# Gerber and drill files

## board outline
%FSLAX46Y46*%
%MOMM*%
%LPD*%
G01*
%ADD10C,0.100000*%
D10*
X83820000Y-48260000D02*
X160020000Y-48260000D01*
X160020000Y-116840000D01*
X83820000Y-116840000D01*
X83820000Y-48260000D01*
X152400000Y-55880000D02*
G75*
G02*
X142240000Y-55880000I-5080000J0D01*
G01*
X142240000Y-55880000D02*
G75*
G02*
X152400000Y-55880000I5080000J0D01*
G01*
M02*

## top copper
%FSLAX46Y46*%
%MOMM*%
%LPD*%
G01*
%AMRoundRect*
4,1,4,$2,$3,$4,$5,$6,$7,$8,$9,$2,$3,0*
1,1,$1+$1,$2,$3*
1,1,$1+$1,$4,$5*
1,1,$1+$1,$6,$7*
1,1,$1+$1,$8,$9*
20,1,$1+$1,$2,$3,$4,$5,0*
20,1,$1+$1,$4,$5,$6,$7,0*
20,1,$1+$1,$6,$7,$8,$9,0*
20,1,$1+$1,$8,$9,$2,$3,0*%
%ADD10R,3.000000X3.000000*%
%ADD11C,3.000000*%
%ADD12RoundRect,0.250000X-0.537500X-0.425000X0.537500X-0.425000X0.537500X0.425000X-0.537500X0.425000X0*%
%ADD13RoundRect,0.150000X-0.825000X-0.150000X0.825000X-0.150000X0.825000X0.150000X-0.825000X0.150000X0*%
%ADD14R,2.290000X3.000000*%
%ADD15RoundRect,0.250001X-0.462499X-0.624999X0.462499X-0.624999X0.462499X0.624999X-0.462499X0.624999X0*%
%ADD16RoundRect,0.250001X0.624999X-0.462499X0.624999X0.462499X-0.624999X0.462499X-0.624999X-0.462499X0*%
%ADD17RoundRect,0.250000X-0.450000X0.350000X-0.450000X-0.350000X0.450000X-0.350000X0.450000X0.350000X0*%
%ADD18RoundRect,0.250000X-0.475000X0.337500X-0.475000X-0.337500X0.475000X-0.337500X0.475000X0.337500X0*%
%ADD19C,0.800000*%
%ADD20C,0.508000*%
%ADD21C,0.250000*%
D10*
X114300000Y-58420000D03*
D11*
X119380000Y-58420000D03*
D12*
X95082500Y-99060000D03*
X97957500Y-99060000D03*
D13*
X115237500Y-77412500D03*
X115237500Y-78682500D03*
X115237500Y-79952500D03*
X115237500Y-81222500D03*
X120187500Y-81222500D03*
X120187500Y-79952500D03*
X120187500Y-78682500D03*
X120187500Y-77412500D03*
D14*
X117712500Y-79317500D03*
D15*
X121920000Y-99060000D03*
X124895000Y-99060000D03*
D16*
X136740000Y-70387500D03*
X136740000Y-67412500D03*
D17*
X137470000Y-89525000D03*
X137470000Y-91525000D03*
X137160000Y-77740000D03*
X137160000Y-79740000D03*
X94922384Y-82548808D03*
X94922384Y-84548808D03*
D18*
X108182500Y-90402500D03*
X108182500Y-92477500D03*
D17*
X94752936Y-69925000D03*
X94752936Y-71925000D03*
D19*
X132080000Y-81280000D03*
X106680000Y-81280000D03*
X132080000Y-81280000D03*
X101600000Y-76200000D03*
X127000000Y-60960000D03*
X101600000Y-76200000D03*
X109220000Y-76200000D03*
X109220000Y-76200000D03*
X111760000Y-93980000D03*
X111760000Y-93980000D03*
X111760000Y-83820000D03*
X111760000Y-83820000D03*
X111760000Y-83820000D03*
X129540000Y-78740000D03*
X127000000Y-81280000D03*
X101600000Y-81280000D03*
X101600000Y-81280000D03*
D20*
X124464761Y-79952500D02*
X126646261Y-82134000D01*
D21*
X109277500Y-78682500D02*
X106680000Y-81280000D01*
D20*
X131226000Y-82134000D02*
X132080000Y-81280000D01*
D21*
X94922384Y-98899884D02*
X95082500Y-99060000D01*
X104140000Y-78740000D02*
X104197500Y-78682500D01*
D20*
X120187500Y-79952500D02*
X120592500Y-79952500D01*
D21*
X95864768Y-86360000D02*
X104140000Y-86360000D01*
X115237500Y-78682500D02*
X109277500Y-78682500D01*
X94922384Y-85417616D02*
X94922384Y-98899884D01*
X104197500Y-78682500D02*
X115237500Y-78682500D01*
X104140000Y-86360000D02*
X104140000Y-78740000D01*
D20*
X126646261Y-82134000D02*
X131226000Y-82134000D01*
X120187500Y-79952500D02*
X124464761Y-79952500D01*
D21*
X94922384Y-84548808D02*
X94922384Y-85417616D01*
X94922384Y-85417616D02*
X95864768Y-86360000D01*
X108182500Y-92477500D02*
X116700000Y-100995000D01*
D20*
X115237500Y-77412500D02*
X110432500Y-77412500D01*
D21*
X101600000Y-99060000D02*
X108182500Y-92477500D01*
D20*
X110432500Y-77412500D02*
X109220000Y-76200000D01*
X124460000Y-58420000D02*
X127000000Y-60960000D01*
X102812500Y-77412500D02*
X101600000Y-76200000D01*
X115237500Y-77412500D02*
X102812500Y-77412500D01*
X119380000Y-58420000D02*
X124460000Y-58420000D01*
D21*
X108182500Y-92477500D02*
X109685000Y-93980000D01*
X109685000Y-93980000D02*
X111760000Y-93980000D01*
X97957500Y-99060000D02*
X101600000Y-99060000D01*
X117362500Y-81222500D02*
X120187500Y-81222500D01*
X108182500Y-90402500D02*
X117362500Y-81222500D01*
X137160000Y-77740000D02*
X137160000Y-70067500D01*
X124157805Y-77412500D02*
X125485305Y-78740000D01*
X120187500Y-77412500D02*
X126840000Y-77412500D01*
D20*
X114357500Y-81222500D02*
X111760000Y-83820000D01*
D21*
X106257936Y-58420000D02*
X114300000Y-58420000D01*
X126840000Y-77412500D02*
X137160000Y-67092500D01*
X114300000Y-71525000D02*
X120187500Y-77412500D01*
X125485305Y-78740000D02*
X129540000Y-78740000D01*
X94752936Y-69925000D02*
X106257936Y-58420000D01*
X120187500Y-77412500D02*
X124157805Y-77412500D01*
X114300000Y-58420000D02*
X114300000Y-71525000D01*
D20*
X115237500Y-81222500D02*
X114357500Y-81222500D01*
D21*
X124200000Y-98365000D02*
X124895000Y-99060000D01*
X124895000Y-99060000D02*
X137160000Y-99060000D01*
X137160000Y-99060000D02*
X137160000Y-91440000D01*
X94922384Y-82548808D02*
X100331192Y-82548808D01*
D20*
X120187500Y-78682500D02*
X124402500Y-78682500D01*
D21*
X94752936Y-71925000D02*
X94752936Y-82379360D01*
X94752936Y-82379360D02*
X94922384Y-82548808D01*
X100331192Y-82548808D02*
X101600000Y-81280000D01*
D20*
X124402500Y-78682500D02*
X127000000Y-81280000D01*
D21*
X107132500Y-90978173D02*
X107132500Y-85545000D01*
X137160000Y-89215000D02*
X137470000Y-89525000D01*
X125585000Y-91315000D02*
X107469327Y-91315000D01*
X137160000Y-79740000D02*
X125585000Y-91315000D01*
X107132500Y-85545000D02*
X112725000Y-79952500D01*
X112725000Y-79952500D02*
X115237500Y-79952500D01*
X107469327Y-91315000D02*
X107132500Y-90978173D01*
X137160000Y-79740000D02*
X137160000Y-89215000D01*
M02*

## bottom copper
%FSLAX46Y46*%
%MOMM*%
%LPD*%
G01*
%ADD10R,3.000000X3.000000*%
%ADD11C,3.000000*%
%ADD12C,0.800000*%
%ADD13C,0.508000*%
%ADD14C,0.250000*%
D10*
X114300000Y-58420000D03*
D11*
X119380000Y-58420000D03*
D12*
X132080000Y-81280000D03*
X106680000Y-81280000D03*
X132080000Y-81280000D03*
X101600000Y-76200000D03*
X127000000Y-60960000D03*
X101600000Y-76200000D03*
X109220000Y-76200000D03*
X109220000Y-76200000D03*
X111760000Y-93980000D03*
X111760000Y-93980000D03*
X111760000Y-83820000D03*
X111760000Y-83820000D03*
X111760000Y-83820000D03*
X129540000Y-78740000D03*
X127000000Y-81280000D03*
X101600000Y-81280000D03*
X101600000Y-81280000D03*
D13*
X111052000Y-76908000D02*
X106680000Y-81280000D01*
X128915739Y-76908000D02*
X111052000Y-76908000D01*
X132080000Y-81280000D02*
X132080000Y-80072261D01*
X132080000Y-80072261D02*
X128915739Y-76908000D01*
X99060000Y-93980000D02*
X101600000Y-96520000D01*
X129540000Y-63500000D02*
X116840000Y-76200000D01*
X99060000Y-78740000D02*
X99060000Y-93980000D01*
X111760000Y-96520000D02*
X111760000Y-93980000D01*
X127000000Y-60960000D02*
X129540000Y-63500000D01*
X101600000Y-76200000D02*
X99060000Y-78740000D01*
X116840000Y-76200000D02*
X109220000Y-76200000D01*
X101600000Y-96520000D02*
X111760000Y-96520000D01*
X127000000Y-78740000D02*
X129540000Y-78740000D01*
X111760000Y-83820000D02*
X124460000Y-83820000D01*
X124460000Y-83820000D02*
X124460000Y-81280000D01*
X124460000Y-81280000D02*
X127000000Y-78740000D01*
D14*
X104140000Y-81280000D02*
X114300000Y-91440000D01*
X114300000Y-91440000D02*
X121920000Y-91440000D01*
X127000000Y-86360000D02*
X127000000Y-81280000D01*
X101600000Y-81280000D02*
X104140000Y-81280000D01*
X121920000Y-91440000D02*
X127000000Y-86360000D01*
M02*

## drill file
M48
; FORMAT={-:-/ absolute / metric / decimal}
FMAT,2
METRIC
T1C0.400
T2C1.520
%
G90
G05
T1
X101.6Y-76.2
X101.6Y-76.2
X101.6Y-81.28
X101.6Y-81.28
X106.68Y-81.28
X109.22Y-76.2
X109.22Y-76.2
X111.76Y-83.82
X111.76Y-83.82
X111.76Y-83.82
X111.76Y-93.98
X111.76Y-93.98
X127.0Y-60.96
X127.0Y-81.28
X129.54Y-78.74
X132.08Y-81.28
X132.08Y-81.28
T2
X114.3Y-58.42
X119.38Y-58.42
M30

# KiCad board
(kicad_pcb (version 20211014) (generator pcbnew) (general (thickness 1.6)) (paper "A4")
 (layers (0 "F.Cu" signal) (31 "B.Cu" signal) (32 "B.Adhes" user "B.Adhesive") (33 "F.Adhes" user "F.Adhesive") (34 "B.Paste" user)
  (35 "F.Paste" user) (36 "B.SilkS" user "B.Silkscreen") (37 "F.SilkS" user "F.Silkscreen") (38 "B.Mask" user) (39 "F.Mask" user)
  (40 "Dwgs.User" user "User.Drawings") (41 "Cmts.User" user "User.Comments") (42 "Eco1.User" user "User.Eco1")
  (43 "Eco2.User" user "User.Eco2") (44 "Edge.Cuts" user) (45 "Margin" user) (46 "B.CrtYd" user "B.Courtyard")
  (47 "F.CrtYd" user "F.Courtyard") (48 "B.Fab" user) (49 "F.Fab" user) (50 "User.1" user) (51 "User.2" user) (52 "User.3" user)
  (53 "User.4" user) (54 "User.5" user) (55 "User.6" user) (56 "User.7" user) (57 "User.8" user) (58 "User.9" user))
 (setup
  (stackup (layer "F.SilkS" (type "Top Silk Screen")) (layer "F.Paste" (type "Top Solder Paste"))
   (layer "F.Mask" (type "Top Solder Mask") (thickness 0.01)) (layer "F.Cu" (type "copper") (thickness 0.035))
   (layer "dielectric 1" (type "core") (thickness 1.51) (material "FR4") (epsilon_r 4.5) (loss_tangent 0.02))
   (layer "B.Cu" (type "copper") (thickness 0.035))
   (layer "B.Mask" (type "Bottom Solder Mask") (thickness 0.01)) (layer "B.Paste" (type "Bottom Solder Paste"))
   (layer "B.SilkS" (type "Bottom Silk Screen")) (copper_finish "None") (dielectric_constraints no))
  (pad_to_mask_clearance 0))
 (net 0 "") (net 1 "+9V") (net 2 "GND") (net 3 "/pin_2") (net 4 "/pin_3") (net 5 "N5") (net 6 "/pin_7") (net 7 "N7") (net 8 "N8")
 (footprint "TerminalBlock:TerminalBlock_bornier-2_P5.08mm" (layer "F.Cu") (at 114.3 58.42)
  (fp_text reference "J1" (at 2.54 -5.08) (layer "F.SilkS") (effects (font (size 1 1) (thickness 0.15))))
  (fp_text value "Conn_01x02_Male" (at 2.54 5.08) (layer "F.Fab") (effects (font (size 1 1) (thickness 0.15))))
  (pad "1" thru_hole rect (at 0 0) (size 3 3) (drill 1.52) (layers *.Cu *.Mask) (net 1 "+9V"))
  (pad "2" thru_hole circle (at 5.08 0) (size 3 3) (drill 1.52) (layers *.Cu *.Mask) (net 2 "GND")))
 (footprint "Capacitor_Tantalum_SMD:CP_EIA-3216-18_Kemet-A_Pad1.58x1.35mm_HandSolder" (layer "F.Cu") (at 96.52 99.06)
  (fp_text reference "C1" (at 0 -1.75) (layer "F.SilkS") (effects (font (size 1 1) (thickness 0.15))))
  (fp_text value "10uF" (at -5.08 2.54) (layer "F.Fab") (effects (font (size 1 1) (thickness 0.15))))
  (pad "1" smd roundrect (at -1.4375 0) (size 1.575 1.35) (layers "F.Cu" "F.Paste" "F.Mask") (roundrect_rratio 0.185185) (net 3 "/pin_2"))
  (pad "2" smd roundrect (at 1.4375 0) (size 1.575 1.35) (layers "F.Cu" "F.Paste" "F.Mask") (roundrect_rratio 0.185185) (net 2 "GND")))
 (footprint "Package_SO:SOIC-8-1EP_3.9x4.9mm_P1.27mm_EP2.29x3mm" (layer "F.Cu") (at 117.7125 79.3175)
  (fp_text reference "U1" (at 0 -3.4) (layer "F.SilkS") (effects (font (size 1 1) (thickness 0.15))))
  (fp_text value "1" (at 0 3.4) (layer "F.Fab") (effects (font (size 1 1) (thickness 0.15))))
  (pad "" smd roundrect (at 0.57 0.75) (size 0.92 1.21) (layers "F.Paste") (roundrect_rratio 0.25))
  (pad "" smd roundrect (at -0.57 -0.75) (size 0.92 1.21) (layers "F.Paste") (roundrect_rratio 0.25))
  (pad "" smd roundrect (at -0.57 0.75) (size 0.92 1.21) (layers "F.Paste") (roundrect_rratio 0.25))
  (pad "" smd roundrect (at 0.57 -0.75) (size 0.92 1.21) (layers "F.Paste") (roundrect_rratio 0.25))
  (pad "1" smd roundrect (at -2.475 -1.905) (size 1.95 0.6) (layers "F.Cu" "F.Paste" "F.Mask") (roundrect_rratio 0.25) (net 2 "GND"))
  (pad "2" smd roundrect (at -2.475 -0.635) (size 1.95 0.6) (layers "F.Cu" "F.Paste" "F.Mask") (roundrect_rratio 0.25) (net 3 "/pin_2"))
  (pad "3" smd roundrect (at -2.475 0.635) (size 1.95 0.6) (layers "F.Cu" "F.Paste" "F.Mask") (roundrect_rratio 0.25) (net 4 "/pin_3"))
  (pad "4" smd roundrect (at -2.475 1.905) (size 1.95 0.6) (layers "F.Cu" "F.Paste" "F.Mask") (roundrect_rratio 0.25) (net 1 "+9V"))
  (pad "5" smd roundrect (at 2.475 1.905) (size 1.95 0.6) (layers "F.Cu" "F.Paste" "F.Mask") (roundrect_rratio 0.25) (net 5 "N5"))
  (pad "6" smd roundrect (at 2.475 0.635) (size 1.95 0.6) (layers "F.Cu" "F.Paste" "F.Mask") (roundrect_rratio 0.25) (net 3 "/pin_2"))
  (pad "7" smd roundrect (at 2.475 -0.635) (size 1.95 0.6) (layers "F.Cu" "F.Paste" "F.Mask") (roundrect_rratio 0.25) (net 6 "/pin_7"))
  (pad "8" smd roundrect (at 2.475 -1.905) (size 1.95 0.6) (layers "F.Cu" "F.Paste" "F.Mask") (roundrect_rratio 0.25) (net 1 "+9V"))
  (pad "9" smd rect (at 0 0) (size 2.29 3) (layers "F.Cu" "F.Mask")))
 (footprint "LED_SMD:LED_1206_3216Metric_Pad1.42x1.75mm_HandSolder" (layer "F.Cu") (at 123.4075 99.06)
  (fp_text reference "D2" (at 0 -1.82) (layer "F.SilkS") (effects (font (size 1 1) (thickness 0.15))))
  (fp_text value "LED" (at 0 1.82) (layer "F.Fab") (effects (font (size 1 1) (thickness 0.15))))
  (pad "1" smd roundrect (at -1.4875 0) (size 1.425 1.75) (layers "F.Cu" "F.Paste" "F.Mask") (roundrect_rratio 0.175439) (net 2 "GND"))
  (pad "2" smd roundrect (at 1.4875 0) (size 1.425 1.75) (layers "F.Cu" "F.Paste" "F.Mask") (roundrect_rratio 0.175439) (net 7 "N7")))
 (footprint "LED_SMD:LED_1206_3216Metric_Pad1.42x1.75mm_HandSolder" (layer "F.Cu") (at 136.74 68.9 90)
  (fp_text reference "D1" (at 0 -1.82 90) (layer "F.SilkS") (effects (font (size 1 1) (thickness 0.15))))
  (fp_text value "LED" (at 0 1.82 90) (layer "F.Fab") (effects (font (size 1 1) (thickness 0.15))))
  (pad "1" smd roundrect (at -1.4875 0 90) (size 1.425 1.75) (layers "F.Cu" "F.Paste" "F.Mask") (roundrect_rratio 0.175439) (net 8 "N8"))
  (pad "2" smd roundrect (at 1.4875 0 90) (size 1.425 1.75) (layers "F.Cu" "F.Paste" "F.Mask") (roundrect_rratio 0.175439) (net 1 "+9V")))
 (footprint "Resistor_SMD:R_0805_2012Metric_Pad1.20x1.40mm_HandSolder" (layer "F.Cu") (at 137.47 90.525 -90)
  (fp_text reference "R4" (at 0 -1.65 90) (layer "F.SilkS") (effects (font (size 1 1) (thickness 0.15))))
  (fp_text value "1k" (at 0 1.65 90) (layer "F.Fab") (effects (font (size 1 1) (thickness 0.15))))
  (pad "1" smd roundrect (at -1 0 270) (size 1.2 1.4) (layers "F.Cu" "F.Paste" "F.Mask") (roundrect_rratio 0.208333) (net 4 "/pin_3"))
  (pad "2" smd roundrect (at 1 0 270) (size 1.2 1.4) (layers "F.Cu" "F.Paste" "F.Mask") (roundrect_rratio 0.208333) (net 7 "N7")))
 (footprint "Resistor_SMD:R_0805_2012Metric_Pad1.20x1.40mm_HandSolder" (layer "F.Cu") (at 137.16 78.74 -90)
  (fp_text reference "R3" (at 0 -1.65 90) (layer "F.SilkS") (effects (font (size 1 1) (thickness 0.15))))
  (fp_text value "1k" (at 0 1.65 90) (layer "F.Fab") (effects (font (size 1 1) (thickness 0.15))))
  (pad "1" smd roundrect (at -1 0 270) (size 1.2 1.4) (layers "F.Cu" "F.Paste" "F.Mask") (roundrect_rratio 0.208333) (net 8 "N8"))
  (pad "2" smd roundrect (at 1 0 270) (size 1.2 1.4) (layers "F.Cu" "F.Paste" "F.Mask") (roundrect_rratio 0.208333) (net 4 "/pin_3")))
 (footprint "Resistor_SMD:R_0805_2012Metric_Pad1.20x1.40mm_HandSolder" (layer "F.Cu") (at 94.922384 83.548808 -90)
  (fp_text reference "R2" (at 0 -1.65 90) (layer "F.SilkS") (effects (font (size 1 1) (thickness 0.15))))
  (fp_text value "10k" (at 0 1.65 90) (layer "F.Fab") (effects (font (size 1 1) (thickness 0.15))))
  (pad "1" smd roundrect (at -1 0 270) (size 1.2 1.4) (layers "F.Cu" "F.Paste" "F.Mask") (roundrect_rratio 0.208333) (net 6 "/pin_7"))
  (pad "2" smd roundrect (at 1 0 270) (size 1.2 1.4) (layers "F.Cu" "F.Paste" "F.Mask") (roundrect_rratio 0.208333) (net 3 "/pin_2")))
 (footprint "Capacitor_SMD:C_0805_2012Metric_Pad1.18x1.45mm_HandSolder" (layer "F.Cu") (at 108.1825 91.44 -90)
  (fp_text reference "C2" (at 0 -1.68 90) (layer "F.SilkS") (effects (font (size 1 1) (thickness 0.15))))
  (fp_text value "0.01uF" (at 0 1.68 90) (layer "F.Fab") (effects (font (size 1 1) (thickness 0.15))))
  (pad "1" smd roundrect (at -1.0375 0 270) (size 1.175 1.45) (layers "F.Cu" "F.Paste" "F.Mask") (roundrect_rratio 0.212766) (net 5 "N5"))
  (pad "2" smd roundrect (at 1.0375 0 270) (size 1.175 1.45) (layers "F.Cu" "F.Paste" "F.Mask") (roundrect_rratio 0.212766) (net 2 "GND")))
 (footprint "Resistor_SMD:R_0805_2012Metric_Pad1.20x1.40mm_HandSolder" (layer "F.Cu") (at 94.752936 70.925 -90)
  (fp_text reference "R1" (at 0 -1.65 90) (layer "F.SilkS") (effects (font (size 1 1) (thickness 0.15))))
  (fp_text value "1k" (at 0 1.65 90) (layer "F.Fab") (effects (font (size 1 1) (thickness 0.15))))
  (pad "1" smd roundrect (at -1 0 270) (size 1.2 1.4) (layers "F.Cu" "F.Paste" "F.Mask") (roundrect_rratio 0.208333) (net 1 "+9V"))
  (pad "2" smd roundrect (at 1 0 270) (size 1.2 1.4) (layers "F.Cu" "F.Paste" "F.Mask") (roundrect_rratio 0.208333) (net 6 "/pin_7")))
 (gr_rect (start 83.82 48.26) (end 160.02 116.84) (layer "Edge.Cuts") (width 0.1) (fill none))
 (gr_circle (center 147.32 55.88) (end 152.4 55.88) (layer "Edge.Cuts") (width 0.1) (fill none))
 (segment (start 124.464761 79.9525) (end 126.646261 82.134) (width 0.508) (layer "F.Cu") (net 3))
 (segment (start 109.2775 78.6825) (end 106.68 81.28) (width 0.25) (layer "F.Cu") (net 3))
 (segment (start 131.226 82.134) (end 132.08 81.28) (width 0.508) (layer "F.Cu") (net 3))
 (segment (start 94.922384 98.899884) (end 95.0825 99.06) (width 0.25) (layer "F.Cu") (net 3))
 (segment (start 104.14 78.74) (end 104.1975 78.6825) (width 0.25) (layer "F.Cu") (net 3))
 (segment (start 120.1875 79.9525) (end 120.5925 79.9525) (width 0.508) (layer "F.Cu") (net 3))
 (segment (start 95.864768 86.36) (end 104.14 86.36) (width 0.25) (layer "F.Cu") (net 3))
 (segment (start 115.2375 78.6825) (end 109.2775 78.6825) (width 0.25) (layer "F.Cu") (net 3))
 (segment (start 94.922384 85.417616) (end 94.922384 98.899884) (width 0.25) (layer "F.Cu") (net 3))
 (segment (start 104.1975 78.6825) (end 115.2375 78.6825) (width 0.25) (layer "F.Cu") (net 3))
 (segment (start 104.14 86.36) (end 104.14 78.74) (width 0.25) (layer "F.Cu") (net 3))
 (segment (start 126.646261 82.134) (end 131.226 82.134) (width 0.508) (layer "F.Cu") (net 3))
 (segment (start 120.1875 79.9525) (end 124.464761 79.9525) (width 0.508) (layer "F.Cu") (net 3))
 (segment (start 94.922384 84.548808) (end 94.922384 85.417616) (width 0.25) (layer "F.Cu") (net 3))
 (segment (start 94.922384 85.417616) (end 95.864768 86.36) (width 0.25) (layer "F.Cu") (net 3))
 (via (at 132.08 81.28) (size 0.8) (drill 0.4) (layers "F.Cu" "B.Cu") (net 3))
 (via (at 106.68 81.28) (size 0.8) (drill 0.4) (layers "F.Cu" "B.Cu") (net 3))
 (via (at 132.08 81.28) (size 0.8) (drill 0.4) (layers "F.Cu" "B.Cu") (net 3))
 (segment (start 111.052 76.908) (end 106.68 81.28) (width 0.508) (layer "B.Cu") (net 3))
 (segment (start 128.915739 76.908) (end 111.052 76.908) (width 0.508) (layer "B.Cu") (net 3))
 (segment (start 132.08 81.28) (end 132.08 80.072261) (width 0.508) (layer "B.Cu") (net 3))
 (segment (start 132.08 80.072261) (end 128.915739 76.908) (width 0.508) (layer "B.Cu") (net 3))
 (segment (start 108.1825 92.4775) (end 116.7 100.995) (width 0.25) (layer "F.Cu") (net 2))
 (segment (start 115.2375 77.4125) (end 110.4325 77.4125) (width 0.508) (layer "F.Cu") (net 2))
 (segment (start 101.6 99.06) (end 108.1825 92.4775) (width 0.25) (layer "F.Cu") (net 2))
 (segment (start 110.4325 77.4125) (end 109.22 76.2) (width 0.508) (layer "F.Cu") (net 2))
 (segment (start 124.46 58.42) (end 127 60.96) (width 0.508) (layer "F.Cu") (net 2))
 (segment (start 102.8125 77.4125) (end 101.6 76.2) (width 0.508) (layer "F.Cu") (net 2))
 (segment (start 115.2375 77.4125) (end 102.8125 77.4125) (width 0.508) (layer "F.Cu") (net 2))
 (segment (start 119.38 58.42) (end 124.46 58.42) (width 0.508) (layer "F.Cu") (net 2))
 (segment (start 108.1825 92.4775) (end 109.685 93.98) (width 0.25) (layer "F.Cu") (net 2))
 (segment (start 109.685 93.98) (end 111.76 93.98) (width 0.25) (layer "F.Cu") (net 2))
 (segment (start 97.9575 99.06) (end 101.6 99.06) (width 0.25) (layer "F.Cu") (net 2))
 (via (at 101.6 76.2) (size 0.8) (drill 0.4) (layers "F.Cu" "B.Cu") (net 2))
 (via (at 127 60.96) (size 0.8) (drill 0.4) (layers "F.Cu" "B.Cu") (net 2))
 (via (at 101.6 76.2) (size 0.8) (drill 0.4) (layers "F.Cu" "B.Cu") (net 2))
 (via (at 109.22 76.2) (size 0.8) (drill 0.4) (layers "F.Cu" "B.Cu") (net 2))
 (via (at 109.22 76.2) (size 0.8) (drill 0.4) (layers "F.Cu" "B.Cu") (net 2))
 (via (at 111.76 93.98) (size 0.8) (drill 0.4) (layers "F.Cu" "B.Cu") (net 2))
 (via (at 111.76 93.98) (size 0.8) (drill 0.4) (layers "F.Cu" "B.Cu") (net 2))
 (segment (start 99.06 93.98) (end 101.6 96.52) (width 0.508) (layer "B.Cu") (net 2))
 (segment (start 129.54 63.5) (end 116.84 76.2) (width 0.508) (layer "B.Cu") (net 2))
 (segment (start 99.06 78.74) (end 99.06 93.98) (width 0.508) (layer "B.Cu") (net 2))
 (segment (start 111.76 96.52) (end 111.76 93.98) (width 0.508) (layer "B.Cu") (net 2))
 (segment (start 127 60.96) (end 129.54 63.5) (width 0.508) (layer "B.Cu") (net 2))
 (segment (start 101.6 76.2) (end 99.06 78.74) (width 0.508) (layer "B.Cu") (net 2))
 (segment (start 116.84 76.2) (end 109.22 76.2) (width 0.508) (layer "B.Cu") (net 2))
 (segment (start 101.6 96.52) (end 111.76 96.52) (width 0.508) (layer "B.Cu") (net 2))
 (segment (start 117.3625 81.2225) (end 120.1875 81.2225) (width 0.25) (layer "F.Cu") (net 5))
 (segment (start 108.1825 90.4025) (end 117.3625 81.2225) (width 0.25) (layer "F.Cu") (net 5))
 (segment (start 137.16 77.74) (end 137.16 70.0675) (width 0.25) (layer "F.Cu") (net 8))
 (segment (start 124.157805 77.4125) (end 125.485305 78.74) (width 0.25) (layer "F.Cu") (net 1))
 (segment (start 120.1875 77.4125) (end 126.84 77.4125) (width 0.25) (layer "F.Cu") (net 1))
 (segment (start 114.3575 81.2225) (end 111.76 83.82) (width 0.508) (layer "F.Cu") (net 1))
 (segment (start 106.257936 58.42) (end 114.3 58.42) (width 0.25) (layer "F.Cu") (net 1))
 (segment (start 126.84 77.4125) (end 137.16 67.0925) (width 0.25) (layer "F.Cu") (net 1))
 (segment (start 114.3 71.525) (end 120.1875 77.4125) (width 0.25) (layer "F.Cu") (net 1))
 (segment (start 125.485305 78.74) (end 129.54 78.74) (width 0.25) (layer "F.Cu") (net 1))
 (segment (start 94.752936 69.925) (end 106.257936 58.42) (width 0.25) (layer "F.Cu") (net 1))
 (segment (start 120.1875 77.4125) (end 124.157805 77.4125) (width 0.25) (layer "F.Cu") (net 1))
 (segment (start 114.3 58.42) (end 114.3 71.525) (width 0.25) (layer "F.Cu") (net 1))
 (segment (start 115.2375 81.2225) (end 114.3575 81.2225) (width 0.508) (layer "F.Cu") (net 1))
 (via (at 111.76 83.82) (size 0.8) (drill 0.4) (layers "F.Cu" "B.Cu") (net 1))
 (via (at 111.76 83.82) (size 0.8) (drill 0.4) (layers "F.Cu" "B.Cu") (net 1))
 (via (at 111.76 83.82) (size 0.8) (drill 0.4) (layers "F.Cu" "B.Cu") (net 1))
 (via (at 129.54 78.74) (size 0.8) (drill 0.4) (layers "F.Cu" "B.Cu") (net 1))
 (segment (start 127 78.74) (end 129.54 78.74) (width 0.508) (layer "B.Cu") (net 1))
 (segment (start 111.76 83.82) (end 124.46 83.82) (width 0.508) (layer "B.Cu") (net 1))
 (segment (start 124.46 83.82) (end 124.46 81.28) (width 0.508) (layer "B.Cu") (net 1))
 (segment (start 124.46 81.28) (end 127 78.74) (width 0.508) (layer "B.Cu") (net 1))
 (segment (start 124.2 98.365) (end 124.895 99.06) (width 0.25) (layer "F.Cu") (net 7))
 (segment (start 124.895 99.06) (end 137.16 99.06) (width 0.25) (layer "F.Cu") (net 7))
 (segment (start 137.16 99.06) (end 137.16 91.44) (width 0.25) (layer "F.Cu") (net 7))
 (segment (start 94.922384 82.548808) (end 100.331192 82.548808) (width 0.25) (layer "F.Cu") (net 6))
 (segment (start 120.1875 78.6825) (end 124.4025 78.6825) (width 0.508) (layer "F.Cu") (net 6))
 (segment (start 94.752936 71.925) (end 94.752936 82.37936) (width 0.25) (layer "F.Cu") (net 6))
 (segment (start 94.752936 82.37936) (end 94.922384 82.548808) (width 0.25) (layer "F.Cu") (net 6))
 (segment (start 100.331192 82.548808) (end 101.6 81.28) (width 0.25) (layer "F.Cu") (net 6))
 (segment (start 124.4025 78.6825) (end 127 81.28) (width 0.508) (layer "F.Cu") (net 6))
 (via (at 127 81.28) (size 0.8) (drill 0.4) (layers "F.Cu" "B.Cu") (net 6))
 (via (at 101.6 81.28) (size 0.8) (drill 0.4) (layers "F.Cu" "B.Cu") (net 6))
 (via (at 101.6 81.28) (size 0.8) (drill 0.4) (layers "F.Cu" "B.Cu") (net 6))
 (segment (start 104.14 81.28) (end 114.3 91.44) (width 0.25) (layer "B.Cu") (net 6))
 (segment (start 114.3 91.44) (end 121.92 91.44) (width 0.25) (layer "B.Cu") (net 6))
 (segment (start 127 86.36) (end 127 81.28) (width 0.25) (layer "B.Cu") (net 6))
 (segment (start 101.6 81.28) (end 104.14 81.28) (width 0.25) (layer "B.Cu") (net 6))
 (segment (start 121.92 91.44) (end 127 86.36) (width 0.25) (layer "B.Cu") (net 6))
 (segment (start 107.1325 90.978173) (end 107.1325 85.545) (width 0.25) (layer "F.Cu") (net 4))
 (segment (start 137.16 89.215) (end 137.47 89.525) (width 0.25) (layer "F.Cu") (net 4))
 (segment (start 125.585 91.315) (end 107.469327 91.315) (width 0.25) (layer "F.Cu") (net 4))
 (segment (start 137.16 79.74) (end 125.585 91.315) (width 0.25) (layer "F.Cu") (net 4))
 (segment (start 107.1325 85.545) (end 112.725 79.9525) (width 0.25) (layer "F.Cu") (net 4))
 (segment (start 112.725 79.9525) (end 115.2375 79.9525) (width 0.25) (layer "F.Cu") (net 4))
 (segment (start 107.469327 91.315) (end 107.1325 90.978173) (width 0.25) (layer "F.Cu") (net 4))
 (segment (start 137.16 79.74) (end 137.16 89.215) (width 0.25) (layer "F.Cu") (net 4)))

